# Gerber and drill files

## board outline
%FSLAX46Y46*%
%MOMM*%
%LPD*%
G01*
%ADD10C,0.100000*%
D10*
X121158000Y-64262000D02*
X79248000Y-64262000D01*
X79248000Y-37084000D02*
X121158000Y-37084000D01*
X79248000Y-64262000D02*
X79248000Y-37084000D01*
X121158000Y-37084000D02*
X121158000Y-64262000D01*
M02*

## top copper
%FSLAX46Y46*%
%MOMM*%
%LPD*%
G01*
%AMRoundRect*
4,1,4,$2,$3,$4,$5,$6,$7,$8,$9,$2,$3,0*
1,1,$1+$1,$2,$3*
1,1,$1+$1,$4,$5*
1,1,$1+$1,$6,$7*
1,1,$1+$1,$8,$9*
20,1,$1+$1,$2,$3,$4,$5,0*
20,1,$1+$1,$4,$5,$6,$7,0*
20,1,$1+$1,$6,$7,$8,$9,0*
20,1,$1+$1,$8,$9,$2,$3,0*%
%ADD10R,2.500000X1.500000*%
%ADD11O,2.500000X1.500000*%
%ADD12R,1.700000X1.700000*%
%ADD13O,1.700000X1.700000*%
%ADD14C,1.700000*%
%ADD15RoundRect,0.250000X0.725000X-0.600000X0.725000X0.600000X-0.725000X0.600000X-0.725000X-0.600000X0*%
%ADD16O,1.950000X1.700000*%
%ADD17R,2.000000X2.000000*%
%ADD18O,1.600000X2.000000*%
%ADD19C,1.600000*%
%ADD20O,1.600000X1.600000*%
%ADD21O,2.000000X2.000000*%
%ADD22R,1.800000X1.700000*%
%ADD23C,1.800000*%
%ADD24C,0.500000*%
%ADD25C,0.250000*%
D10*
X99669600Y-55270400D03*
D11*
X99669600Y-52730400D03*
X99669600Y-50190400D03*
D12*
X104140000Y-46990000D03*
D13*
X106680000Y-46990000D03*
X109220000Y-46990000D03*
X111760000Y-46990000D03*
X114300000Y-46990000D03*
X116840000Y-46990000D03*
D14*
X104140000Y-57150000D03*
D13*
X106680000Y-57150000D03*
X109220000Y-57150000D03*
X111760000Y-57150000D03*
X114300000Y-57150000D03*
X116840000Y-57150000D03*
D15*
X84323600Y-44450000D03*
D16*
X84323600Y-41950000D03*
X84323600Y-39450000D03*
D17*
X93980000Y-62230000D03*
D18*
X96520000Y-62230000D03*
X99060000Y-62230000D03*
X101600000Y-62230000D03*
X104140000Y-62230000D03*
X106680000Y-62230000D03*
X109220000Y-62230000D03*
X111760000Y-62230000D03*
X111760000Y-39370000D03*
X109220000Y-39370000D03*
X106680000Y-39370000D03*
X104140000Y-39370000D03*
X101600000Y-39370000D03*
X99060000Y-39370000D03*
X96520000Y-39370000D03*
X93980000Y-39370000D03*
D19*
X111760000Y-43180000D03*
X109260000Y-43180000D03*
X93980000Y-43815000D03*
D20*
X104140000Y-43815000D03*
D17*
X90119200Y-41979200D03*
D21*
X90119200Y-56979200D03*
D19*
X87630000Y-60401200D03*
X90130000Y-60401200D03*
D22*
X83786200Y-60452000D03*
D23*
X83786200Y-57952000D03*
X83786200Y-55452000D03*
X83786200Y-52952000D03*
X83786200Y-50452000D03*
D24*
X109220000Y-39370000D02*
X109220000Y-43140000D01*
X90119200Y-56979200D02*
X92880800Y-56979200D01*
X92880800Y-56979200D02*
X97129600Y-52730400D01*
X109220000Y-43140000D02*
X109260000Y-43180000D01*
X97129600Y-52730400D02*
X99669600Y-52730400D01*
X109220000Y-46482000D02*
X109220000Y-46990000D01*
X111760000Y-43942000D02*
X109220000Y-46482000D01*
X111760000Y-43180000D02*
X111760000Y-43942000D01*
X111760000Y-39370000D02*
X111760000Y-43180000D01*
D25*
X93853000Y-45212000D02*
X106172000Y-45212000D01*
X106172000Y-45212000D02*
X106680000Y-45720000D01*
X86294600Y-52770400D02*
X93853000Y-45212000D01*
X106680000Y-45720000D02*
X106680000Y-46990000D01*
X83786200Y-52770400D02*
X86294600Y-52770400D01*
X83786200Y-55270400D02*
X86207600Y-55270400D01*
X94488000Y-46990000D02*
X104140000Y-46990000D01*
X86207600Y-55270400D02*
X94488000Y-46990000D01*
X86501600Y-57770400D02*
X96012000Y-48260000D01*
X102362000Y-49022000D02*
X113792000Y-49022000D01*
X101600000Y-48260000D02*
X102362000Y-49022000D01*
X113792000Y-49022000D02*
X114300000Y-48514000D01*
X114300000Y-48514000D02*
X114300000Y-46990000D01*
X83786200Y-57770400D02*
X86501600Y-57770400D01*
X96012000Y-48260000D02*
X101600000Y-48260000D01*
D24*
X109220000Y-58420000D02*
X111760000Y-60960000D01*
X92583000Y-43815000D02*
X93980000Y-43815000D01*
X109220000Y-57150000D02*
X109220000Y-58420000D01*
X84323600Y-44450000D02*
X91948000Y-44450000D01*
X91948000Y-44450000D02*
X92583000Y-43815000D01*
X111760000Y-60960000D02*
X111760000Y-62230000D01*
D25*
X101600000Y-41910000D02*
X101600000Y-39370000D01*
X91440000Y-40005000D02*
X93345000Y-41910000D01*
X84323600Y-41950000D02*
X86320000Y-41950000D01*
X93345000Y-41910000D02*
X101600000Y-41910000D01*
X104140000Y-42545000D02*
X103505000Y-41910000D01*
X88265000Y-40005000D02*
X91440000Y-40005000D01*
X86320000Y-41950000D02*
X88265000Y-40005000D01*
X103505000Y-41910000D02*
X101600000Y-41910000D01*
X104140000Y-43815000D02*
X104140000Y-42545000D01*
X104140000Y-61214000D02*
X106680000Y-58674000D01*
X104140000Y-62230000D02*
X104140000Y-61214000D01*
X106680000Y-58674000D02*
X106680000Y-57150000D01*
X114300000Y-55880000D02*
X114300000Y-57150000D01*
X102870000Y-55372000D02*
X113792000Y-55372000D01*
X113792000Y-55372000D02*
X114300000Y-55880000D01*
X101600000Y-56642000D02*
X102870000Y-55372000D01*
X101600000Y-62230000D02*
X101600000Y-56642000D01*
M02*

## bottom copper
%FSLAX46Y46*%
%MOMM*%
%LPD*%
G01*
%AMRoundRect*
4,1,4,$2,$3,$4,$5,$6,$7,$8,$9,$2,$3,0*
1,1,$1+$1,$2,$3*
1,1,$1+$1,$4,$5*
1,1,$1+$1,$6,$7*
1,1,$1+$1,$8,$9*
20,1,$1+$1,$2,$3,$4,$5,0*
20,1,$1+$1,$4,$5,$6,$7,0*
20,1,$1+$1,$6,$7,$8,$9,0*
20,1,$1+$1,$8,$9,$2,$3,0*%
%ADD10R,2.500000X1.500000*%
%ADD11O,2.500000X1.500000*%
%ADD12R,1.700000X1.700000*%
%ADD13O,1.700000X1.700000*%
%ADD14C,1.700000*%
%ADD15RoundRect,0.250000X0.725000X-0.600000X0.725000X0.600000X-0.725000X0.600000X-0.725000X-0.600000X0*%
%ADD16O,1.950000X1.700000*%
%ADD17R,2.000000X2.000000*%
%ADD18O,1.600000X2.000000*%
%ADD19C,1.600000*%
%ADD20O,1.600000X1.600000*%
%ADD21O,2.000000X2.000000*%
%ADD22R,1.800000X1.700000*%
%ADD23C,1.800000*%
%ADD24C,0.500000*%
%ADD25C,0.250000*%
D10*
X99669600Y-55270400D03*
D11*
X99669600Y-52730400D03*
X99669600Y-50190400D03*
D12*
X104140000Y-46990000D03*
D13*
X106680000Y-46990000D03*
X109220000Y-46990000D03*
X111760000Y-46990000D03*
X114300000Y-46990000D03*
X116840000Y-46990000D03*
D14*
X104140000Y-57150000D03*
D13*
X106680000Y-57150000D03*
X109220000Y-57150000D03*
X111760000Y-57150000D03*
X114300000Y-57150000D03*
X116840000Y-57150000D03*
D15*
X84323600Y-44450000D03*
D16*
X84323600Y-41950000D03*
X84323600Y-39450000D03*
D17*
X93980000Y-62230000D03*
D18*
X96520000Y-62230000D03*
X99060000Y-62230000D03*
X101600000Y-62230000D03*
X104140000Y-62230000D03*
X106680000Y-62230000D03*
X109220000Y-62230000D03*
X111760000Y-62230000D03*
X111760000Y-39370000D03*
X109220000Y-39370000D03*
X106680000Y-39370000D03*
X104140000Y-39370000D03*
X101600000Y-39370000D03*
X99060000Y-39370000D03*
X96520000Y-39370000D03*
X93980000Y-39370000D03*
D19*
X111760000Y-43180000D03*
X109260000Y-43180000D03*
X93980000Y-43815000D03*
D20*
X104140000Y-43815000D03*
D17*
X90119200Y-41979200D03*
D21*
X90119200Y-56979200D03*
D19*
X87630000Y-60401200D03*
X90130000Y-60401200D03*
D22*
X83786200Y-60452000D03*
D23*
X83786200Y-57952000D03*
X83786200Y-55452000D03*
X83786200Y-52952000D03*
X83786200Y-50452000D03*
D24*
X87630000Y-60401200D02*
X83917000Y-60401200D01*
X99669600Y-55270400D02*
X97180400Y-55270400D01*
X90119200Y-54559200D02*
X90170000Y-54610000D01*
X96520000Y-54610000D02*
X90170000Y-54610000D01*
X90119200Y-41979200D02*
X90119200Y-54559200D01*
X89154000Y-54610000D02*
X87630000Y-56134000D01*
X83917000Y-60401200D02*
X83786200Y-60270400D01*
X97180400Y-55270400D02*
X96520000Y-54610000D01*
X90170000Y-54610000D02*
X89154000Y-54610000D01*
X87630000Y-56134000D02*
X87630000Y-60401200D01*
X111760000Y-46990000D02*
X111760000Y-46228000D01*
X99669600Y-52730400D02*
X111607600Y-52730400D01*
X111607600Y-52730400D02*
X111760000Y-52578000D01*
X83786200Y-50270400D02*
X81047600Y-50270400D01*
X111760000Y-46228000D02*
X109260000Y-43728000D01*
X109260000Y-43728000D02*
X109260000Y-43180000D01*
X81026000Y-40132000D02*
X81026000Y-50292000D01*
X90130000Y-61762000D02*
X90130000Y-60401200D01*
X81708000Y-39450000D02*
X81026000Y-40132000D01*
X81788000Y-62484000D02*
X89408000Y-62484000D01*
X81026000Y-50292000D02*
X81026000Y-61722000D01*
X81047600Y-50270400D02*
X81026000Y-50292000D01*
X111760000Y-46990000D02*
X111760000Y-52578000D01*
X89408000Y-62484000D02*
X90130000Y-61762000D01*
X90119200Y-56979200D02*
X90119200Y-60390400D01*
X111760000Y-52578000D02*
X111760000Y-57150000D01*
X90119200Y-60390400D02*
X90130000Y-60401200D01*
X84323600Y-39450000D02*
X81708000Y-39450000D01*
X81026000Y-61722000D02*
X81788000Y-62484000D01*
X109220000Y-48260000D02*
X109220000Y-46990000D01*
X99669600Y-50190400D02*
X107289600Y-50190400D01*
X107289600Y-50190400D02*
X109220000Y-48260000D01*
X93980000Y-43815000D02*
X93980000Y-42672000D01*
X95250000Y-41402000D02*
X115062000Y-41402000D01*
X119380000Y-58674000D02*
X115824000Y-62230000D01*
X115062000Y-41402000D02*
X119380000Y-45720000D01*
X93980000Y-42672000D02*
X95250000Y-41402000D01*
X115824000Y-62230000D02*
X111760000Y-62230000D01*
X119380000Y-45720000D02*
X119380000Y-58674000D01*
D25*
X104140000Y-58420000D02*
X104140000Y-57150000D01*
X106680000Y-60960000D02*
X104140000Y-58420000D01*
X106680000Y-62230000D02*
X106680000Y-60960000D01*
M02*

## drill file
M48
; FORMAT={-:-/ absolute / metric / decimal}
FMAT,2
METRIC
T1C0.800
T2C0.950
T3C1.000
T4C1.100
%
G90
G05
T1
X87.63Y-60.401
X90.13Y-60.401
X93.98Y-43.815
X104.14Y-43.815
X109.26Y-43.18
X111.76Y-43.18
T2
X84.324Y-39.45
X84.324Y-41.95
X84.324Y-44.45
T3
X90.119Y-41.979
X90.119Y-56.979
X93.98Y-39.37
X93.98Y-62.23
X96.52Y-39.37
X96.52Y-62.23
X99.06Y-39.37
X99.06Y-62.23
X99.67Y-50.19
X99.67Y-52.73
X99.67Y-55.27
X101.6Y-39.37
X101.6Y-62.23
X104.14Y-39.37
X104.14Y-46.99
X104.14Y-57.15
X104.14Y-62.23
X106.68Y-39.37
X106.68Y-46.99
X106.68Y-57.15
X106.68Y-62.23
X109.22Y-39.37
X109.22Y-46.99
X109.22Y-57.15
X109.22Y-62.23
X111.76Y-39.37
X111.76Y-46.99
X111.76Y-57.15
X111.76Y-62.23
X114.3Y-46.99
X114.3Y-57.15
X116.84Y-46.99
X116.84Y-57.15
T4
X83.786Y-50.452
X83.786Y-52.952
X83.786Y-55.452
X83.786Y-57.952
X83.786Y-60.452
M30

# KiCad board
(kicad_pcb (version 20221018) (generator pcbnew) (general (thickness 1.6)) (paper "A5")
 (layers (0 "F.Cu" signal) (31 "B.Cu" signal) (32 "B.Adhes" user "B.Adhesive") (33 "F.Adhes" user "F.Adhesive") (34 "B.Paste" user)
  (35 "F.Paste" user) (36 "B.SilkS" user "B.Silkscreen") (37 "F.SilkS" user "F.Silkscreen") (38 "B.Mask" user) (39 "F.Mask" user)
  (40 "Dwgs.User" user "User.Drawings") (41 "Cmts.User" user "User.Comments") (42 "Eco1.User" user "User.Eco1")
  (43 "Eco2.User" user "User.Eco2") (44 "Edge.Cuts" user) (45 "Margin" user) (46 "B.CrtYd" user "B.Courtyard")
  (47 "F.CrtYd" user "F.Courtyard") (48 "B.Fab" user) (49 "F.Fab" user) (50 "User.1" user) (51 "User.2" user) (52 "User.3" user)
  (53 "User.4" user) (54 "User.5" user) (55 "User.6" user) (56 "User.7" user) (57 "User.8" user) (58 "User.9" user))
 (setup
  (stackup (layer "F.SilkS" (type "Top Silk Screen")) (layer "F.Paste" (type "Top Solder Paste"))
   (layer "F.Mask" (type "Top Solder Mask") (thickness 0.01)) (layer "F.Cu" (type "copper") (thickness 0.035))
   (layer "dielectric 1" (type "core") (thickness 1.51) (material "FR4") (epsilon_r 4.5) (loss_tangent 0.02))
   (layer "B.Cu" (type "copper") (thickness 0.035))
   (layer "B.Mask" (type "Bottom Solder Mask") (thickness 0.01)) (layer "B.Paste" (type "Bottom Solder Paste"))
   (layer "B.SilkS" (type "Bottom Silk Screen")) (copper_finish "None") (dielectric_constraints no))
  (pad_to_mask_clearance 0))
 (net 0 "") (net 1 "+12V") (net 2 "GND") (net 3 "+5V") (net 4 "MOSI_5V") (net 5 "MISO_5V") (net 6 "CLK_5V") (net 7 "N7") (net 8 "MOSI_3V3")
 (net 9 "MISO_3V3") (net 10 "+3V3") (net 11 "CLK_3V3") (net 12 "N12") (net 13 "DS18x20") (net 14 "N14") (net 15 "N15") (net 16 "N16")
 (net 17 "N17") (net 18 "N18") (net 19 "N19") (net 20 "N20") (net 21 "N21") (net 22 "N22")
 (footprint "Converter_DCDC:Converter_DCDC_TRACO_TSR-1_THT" (layer "F.Cu") (at 99.6696 55.2704 90)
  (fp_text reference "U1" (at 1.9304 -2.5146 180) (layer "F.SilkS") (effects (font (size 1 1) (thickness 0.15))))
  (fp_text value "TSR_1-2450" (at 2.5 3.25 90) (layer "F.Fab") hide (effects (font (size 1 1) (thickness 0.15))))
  (pad "1" thru_hole rect (at 0 0 90) (size 1.5 2.5) (drill 1) (layers "*.Cu" "*.Mask") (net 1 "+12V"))
  (pad "2" thru_hole oval (at 2.54 0 90) (size 1.5 2.5) (drill 1) (layers "*.Cu" "*.Mask") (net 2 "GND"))
  (pad "3" thru_hole oval (at 5.08 0 90) (size 1.5 2.5) (drill 1) (layers "*.Cu" "*.Mask") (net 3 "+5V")))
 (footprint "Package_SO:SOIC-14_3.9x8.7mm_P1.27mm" (layer "F.Cu") (at 110.49 52.07 90)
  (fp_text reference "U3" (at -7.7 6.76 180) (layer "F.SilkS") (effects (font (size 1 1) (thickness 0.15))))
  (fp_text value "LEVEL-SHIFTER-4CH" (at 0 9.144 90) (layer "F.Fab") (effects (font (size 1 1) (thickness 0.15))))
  (pad "1" thru_hole rect (at 5.08 -6.35 90) (size 1.7 1.7) (drill 1) (layers "*.Cu" "*.Mask") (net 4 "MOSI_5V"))
  (pad "2" thru_hole oval (at 5.08 -3.81 90) (size 1.7 1.7) (drill 1) (layers "*.Cu" "*.Mask") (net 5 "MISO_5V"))
  (pad "3" thru_hole oval (at 5.08 -1.27 90) (size 1.7 1.7) (drill 1) (layers "*.Cu" "*.Mask") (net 3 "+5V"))
  (pad "4" thru_hole oval (at 5.08 1.27 90) (size 1.7 1.7) (drill 1) (layers "*.Cu" "*.Mask") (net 2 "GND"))
  (pad "5" thru_hole oval (at 5.08 3.81 90) (size 1.7 1.7) (drill 1) (layers "*.Cu" "*.Mask") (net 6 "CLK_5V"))
  (pad "6" thru_hole oval (at 5.08 6.35 90) (size 1.7 1.7) (drill 1) (layers "*.Cu" "*.Mask") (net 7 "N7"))
  (pad "7" thru_hole circle (at -5.08 -6.35 90) (size 1.7 1.7) (drill 1) (layers "*.Cu" "*.Mask") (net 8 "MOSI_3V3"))
  (pad "8" thru_hole oval (at -5.08 -3.81 90) (size 1.7 1.7) (drill 1) (layers "*.Cu" "*.Mask") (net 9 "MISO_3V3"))
  (pad "9" thru_hole oval (at -5.08 -1.27 90) (size 1.7 1.7) (drill 1) (layers "*.Cu" "*.Mask") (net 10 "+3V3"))
  (pad "10" thru_hole oval (at -5.08 1.27 90) (size 1.7 1.7) (drill 1) (layers "*.Cu" "*.Mask") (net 2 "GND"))
  (pad "11" thru_hole oval (at -5.08 3.81 90) (size 1.7 1.7) (drill 1) (layers "*.Cu" "*.Mask") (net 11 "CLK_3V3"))
  (pad "12" thru_hole oval (at -5.08 6.35 90) (size 1.7 1.7) (drill 1) (layers "*.Cu" "*.Mask") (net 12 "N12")))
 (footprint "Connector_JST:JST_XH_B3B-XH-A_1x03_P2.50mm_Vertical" (layer "F.Cu") (at 84.3236 44.45 90)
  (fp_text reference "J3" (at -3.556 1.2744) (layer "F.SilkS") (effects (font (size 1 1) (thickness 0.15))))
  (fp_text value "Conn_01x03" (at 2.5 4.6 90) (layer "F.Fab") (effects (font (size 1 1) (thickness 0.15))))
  (pad "1" thru_hole roundrect (at 0 0 90) (size 1.7 1.95) (drill 0.95) (layers "*.Cu" "*.Mask") (roundrect_rratio 0.1470588235)
   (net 10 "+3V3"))
  (pad "2" thru_hole oval (at 2.5 0 90) (size 1.7 1.95) (drill 0.95) (layers "*.Cu" "*.Mask") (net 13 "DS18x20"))
  (pad "3" thru_hole oval (at 5 0 90) (size 1.7 1.95) (drill 0.95) (layers "*.Cu" "*.Mask") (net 2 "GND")))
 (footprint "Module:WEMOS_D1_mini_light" (layer "F.Cu") (at 93.98 62.23 90)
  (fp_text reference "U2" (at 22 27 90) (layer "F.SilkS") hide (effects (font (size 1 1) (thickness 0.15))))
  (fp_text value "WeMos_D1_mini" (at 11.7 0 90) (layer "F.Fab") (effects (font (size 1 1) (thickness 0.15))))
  (pad "1" thru_hole rect (at 0 0 90) (size 2 2) (drill 1) (layers "*.Cu" "*.Mask") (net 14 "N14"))
  (pad "2" thru_hole oval (at 0 2.54 90) (size 2 1.6) (drill 1) (layers "*.Cu" "*.Mask") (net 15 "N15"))
  (pad "3" thru_hole oval (at 0 5.08 90) (size 2 1.6) (drill 1) (layers "*.Cu" "*.Mask") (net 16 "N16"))
  (pad "4" thru_hole oval (at 0 7.62 90) (size 2 1.6) (drill 1) (layers "*.Cu" "*.Mask") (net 11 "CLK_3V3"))
  (pad "5" thru_hole oval (at 0 10.16 90) (size 2 1.6) (drill 1) (layers "*.Cu" "*.Mask") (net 9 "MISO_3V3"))
  (pad "6" thru_hole oval (at 0 12.7 90) (size 2 1.6) (drill 1) (layers "*.Cu" "*.Mask") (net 8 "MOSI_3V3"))
  (pad "7" thru_hole oval (at 0 15.24 90) (size 2 1.6) (drill 1) (layers "*.Cu" "*.Mask") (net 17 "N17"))
  (pad "8" thru_hole oval (at 0 17.78 90) (size 2 1.6) (drill 1) (layers "*.Cu" "*.Mask") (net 10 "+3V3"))
  (pad "9" thru_hole oval (at 22.86 17.78 90) (size 2 1.6) (drill 1) (layers "*.Cu" "*.Mask") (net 3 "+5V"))
  (pad "10" thru_hole oval (at 22.86 15.24 90) (size 2 1.6) (drill 1) (layers "*.Cu" "*.Mask") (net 2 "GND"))
  (pad "11" thru_hole oval (at 22.86 12.7 90) (size 2 1.6) (drill 1) (layers "*.Cu" "*.Mask") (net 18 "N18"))
  (pad "12" thru_hole oval (at 22.86 10.16 90) (size 2 1.6) (drill 1) (layers "*.Cu" "*.Mask") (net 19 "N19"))
  (pad "13" thru_hole oval (at 22.86 7.62 90) (size 2 1.6) (drill 1) (layers "*.Cu" "*.Mask") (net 13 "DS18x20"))
  (pad "14" thru_hole oval (at 22.86 5.08 90) (size 2 1.6) (drill 1) (layers "*.Cu" "*.Mask") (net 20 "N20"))
  (pad "15" thru_hole oval (at 22.86 2.54 90) (size 2 1.6) (drill 1) (layers "*.Cu" "*.Mask") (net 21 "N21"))
  (pad "16" thru_hole oval (at 22.86 0 90) (size 2 1.6) (drill 1) (layers "*.Cu" "*.Mask") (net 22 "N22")))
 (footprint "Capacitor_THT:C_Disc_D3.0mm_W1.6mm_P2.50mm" (layer "F.Cu") (at 111.76 43.18 180)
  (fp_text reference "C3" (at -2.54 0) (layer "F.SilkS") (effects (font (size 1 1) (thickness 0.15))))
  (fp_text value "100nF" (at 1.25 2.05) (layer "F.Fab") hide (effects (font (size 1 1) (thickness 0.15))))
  (pad "1" thru_hole circle (at 0 0 180) (size 1.6 1.6) (drill 0.8) (layers "*.Cu" "*.Mask") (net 3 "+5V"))
  (pad "2" thru_hole circle (at 2.5 0 180) (size 1.6 1.6) (drill 0.8) (layers "*.Cu" "*.Mask") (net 2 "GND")))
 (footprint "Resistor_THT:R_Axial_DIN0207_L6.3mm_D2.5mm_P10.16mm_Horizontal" (layer "F.Cu") (at 93.98 43.815)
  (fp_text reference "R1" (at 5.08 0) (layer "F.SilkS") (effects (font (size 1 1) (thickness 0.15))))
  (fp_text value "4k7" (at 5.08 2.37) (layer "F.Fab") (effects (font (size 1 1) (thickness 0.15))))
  (pad "1" thru_hole circle (at 0 0) (size 1.6 1.6) (drill 0.8) (layers "*.Cu" "*.Mask") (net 10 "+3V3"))
  (pad "2" thru_hole oval (at 10.16 0) (size 1.6 1.6) (drill 0.8) (layers "*.Cu" "*.Mask") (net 13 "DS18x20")))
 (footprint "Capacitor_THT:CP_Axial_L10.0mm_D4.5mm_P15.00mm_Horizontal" (layer "F.Cu") (at 90.1192 41.9792 -90)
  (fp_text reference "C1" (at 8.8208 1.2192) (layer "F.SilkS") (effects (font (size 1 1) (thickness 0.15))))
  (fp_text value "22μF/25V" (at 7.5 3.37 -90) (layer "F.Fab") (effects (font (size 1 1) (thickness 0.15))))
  (pad "1" thru_hole rect (at 0 0 270) (size 2 2) (drill 1) (layers "*.Cu" "*.Mask") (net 1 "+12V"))
  (pad "2" thru_hole oval (at 15 0 270) (size 2 2) (drill 1) (layers "*.Cu" "*.Mask") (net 2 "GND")))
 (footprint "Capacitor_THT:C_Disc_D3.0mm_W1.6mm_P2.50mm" (layer "F.Cu") (at 87.63 60.4012)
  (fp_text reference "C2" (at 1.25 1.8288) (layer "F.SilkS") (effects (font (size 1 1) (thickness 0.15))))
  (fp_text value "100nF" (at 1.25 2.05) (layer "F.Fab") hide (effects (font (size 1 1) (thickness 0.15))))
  (pad "1" thru_hole circle (at 0 0) (size 1.6 1.6) (drill 0.8) (layers "*.Cu" "*.Mask") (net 1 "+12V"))
  (pad "2" thru_hole circle (at 2.5 0) (size 1.6 1.6) (drill 0.8) (layers "*.Cu" "*.Mask") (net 2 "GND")))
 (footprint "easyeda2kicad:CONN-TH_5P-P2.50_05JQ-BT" (layer "B.Cu") (at 83.7862 55.452 -90)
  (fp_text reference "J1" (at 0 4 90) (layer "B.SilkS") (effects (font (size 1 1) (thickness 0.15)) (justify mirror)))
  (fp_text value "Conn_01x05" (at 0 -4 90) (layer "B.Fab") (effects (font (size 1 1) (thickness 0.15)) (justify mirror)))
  (pad "1" thru_hole rect (at 5 0 90) (size 1.7 1.8) (drill 1.100023) (layers "*.Cu" "*.Paste" "*.Mask") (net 2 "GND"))
  (pad "2" thru_hole circle (at 2.5 0 90) (size 1.8 1.8) (drill 1.100023) (layers "*.Cu" "*.Paste" "*.Mask") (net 5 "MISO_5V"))
  (pad "3" thru_hole circle (at 0 0 90) (size 1.8 1.8) (drill 1.100023) (layers "*.Cu" "*.Paste" "*.Mask") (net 4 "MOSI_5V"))
  (pad "4" thru_hole circle (at -2.5 0 90) (size 1.8 1.8) (drill 1.100023) (layers "*.Cu" "*.Paste" "*.Mask") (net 6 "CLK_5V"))
  (pad "5" thru_hole circle (at -5 0 90) (size 1.8 1.8) (drill 1.100023) (layers "*.Cu" "*.Paste" "*.Mask") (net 1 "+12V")))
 (gr_line (start 121.158 64.262) (end 79.248 64.262) (stroke (width 0.1) (type solid)) (layer "Edge.Cuts"))
 (gr_line (start 79.248 37.084) (end 121.158 37.084) (stroke (width 0.1) (type solid)) (layer "Edge.Cuts"))
 (gr_line (start 79.248 64.262) (end 79.248 37.084) (stroke (width 0.1) (type solid)) (layer "Edge.Cuts"))
 (gr_line (start 121.158 37.084) (end 121.158 64.262) (stroke (width 0.1) (type solid)) (layer "Edge.Cuts"))
 (segment (start 87.63 60.4012) (end 83.917 60.4012) (width 0.5) (layer "B.Cu") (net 1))
 (segment (start 99.6696 55.2704) (end 97.1804 55.2704) (width 0.5) (layer "B.Cu") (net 1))
 (segment (start 90.1192 54.5592) (end 90.17 54.61) (width 0.5) (layer "B.Cu") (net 1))
 (segment (start 96.52 54.61) (end 90.17 54.61) (width 0.5) (layer "B.Cu") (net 1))
 (segment (start 90.1192 41.9792) (end 90.1192 54.5592) (width 0.5) (layer "B.Cu") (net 1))
 (segment (start 89.154 54.61) (end 87.63 56.134) (width 0.5) (layer "B.Cu") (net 1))
 (segment (start 83.917 60.4012) (end 83.7862 60.2704) (width 0.5) (layer "B.Cu") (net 1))
 (segment (start 97.1804 55.2704) (end 96.52 54.61) (width 0.5) (layer "B.Cu") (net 1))
 (segment (start 90.17 54.61) (end 89.154 54.61) (width 0.5) (layer "B.Cu") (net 1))
 (segment (start 87.63 56.134) (end 87.63 60.4012) (width 0.5) (layer "B.Cu") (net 1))
 (segment (start 109.22 39.37) (end 109.22 43.14) (width 0.5) (layer "F.Cu") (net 2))
 (segment (start 90.1192 56.9792) (end 92.8808 56.9792) (width 0.5) (layer "F.Cu") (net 2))
 (segment (start 92.8808 56.9792) (end 97.1296 52.7304) (width 0.5) (layer "F.Cu") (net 2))
 (segment (start 109.22 43.14) (end 109.26 43.18) (width 0.5) (layer "F.Cu") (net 2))
 (segment (start 97.1296 52.7304) (end 99.6696 52.7304) (width 0.5) (layer "F.Cu") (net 2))
 (segment (start 111.76 46.99) (end 111.76 46.228) (width 0.5) (layer "B.Cu") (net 2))
 (segment (start 99.6696 52.7304) (end 111.6076 52.7304) (width 0.5) (layer "B.Cu") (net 2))
 (segment (start 111.6076 52.7304) (end 111.76 52.578) (width 0.5) (layer "B.Cu") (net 2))
 (segment (start 83.7862 50.2704) (end 81.0476 50.2704) (width 0.5) (layer "B.Cu") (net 2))
 (segment (start 111.76 46.228) (end 109.26 43.728) (width 0.5) (layer "B.Cu") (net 2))
 (segment (start 109.26 43.728) (end 109.26 43.18) (width 0.5) (layer "B.Cu") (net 2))
 (segment (start 81.026 40.132) (end 81.026 50.292) (width 0.5) (layer "B.Cu") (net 2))
 (segment (start 90.13 61.762) (end 90.13 60.4012) (width 0.5) (layer "B.Cu") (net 2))
 (segment (start 81.708 39.45) (end 81.026 40.132) (width 0.5) (layer "B.Cu") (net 2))
 (segment (start 81.788 62.484) (end 89.408 62.484) (width 0.5) (layer "B.Cu") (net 2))
 (segment (start 81.026 50.292) (end 81.026 61.722) (width 0.5) (layer "B.Cu") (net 2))
 (segment (start 81.0476 50.2704) (end 81.026 50.292) (width 0.5) (layer "B.Cu") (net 2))
 (segment (start 111.76 46.99) (end 111.76 52.578) (width 0.5) (layer "B.Cu") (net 2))
 (segment (start 89.408 62.484) (end 90.13 61.762) (width 0.5) (layer "B.Cu") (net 2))
 (segment (start 90.1192 56.9792) (end 90.1192 60.3904) (width 0.5) (layer "B.Cu") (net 2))
 (segment (start 111.76 52.578) (end 111.76 57.15) (width 0.5) (layer "B.Cu") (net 2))
 (segment (start 90.1192 60.3904) (end 90.13 60.4012) (width 0.5) (layer "B.Cu") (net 2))
 (segment (start 84.3236 39.45) (end 81.708 39.45) (width 0.5) (layer "B.Cu") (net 2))
 (segment (start 81.026 61.722) (end 81.788 62.484) (width 0.5) (layer "B.Cu") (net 2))
 (segment (start 109.22 46.482) (end 109.22 46.99) (width 0.5) (layer "F.Cu") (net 3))
 (segment (start 111.76 43.942) (end 109.22 46.482) (width 0.5) (layer "F.Cu") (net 3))
 (segment (start 111.76 43.18) (end 111.76 43.942) (width 0.5) (layer "F.Cu") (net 3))
 (segment (start 111.76 39.37) (end 111.76 43.18) (width 0.5) (layer "F.Cu") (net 3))
 (segment (start 109.22 48.26) (end 109.22 46.99) (width 0.5) (layer "B.Cu") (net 3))
 (segment (start 99.6696 50.1904) (end 107.2896 50.1904) (width 0.5) (layer "B.Cu") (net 3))
 (segment (start 107.2896 50.1904) (end 109.22 48.26) (width 0.5) (layer "B.Cu") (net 3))
 (segment (start 93.853 45.212) (end 106.172 45.212) (width 0.25) (layer "F.Cu") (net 5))
 (segment (start 106.172 45.212) (end 106.68 45.72) (width 0.25) (layer "F.Cu") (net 5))
 (segment (start 86.2946 52.7704) (end 93.853 45.212) (width 0.25) (layer "F.Cu") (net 5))
 (segment (start 106.68 45.72) (end 106.68 46.99) (width 0.25) (layer "F.Cu") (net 5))
 (segment (start 83.7862 52.7704) (end 86.2946 52.7704) (width 0.25) (layer "F.Cu") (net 5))
 (segment (start 83.7862 55.2704) (end 86.2076 55.2704) (width 0.25) (layer "F.Cu") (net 4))
 (segment (start 94.488 46.99) (end 104.14 46.99) (width 0.25) (layer "F.Cu") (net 4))
 (segment (start 86.2076 55.2704) (end 94.488 46.99) (width 0.25) (layer "F.Cu") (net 4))
 (segment (start 86.5016 57.7704) (end 96.012 48.26) (width 0.25) (layer "F.Cu") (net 6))
 (segment (start 102.362 49.022) (end 113.792 49.022) (width 0.25) (layer "F.Cu") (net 6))
 (segment (start 101.6 48.26) (end 102.362 49.022) (width 0.25) (layer "F.Cu") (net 6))
 (segment (start 113.792 49.022) (end 114.3 48.514) (width 0.25) (layer "F.Cu") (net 6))
 (segment (start 114.3 48.514) (end 114.3 46.99) (width 0.25) (layer "F.Cu") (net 6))
 (segment (start 83.7862 57.7704) (end 86.5016 57.7704) (width 0.25) (layer "F.Cu") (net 6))
 (segment (start 96.012 48.26) (end 101.6 48.26) (width 0.25) (layer "F.Cu") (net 6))
 (segment (start 109.22 58.42) (end 111.76 60.96) (width 0.5) (layer "F.Cu") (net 10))
 (segment (start 92.583 43.815) (end 93.98 43.815) (width 0.5) (layer "F.Cu") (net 10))
 (segment (start 109.22 57.15) (end 109.22 58.42) (width 0.5) (layer "F.Cu") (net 10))
 (segment (start 84.3236 44.45) (end 91.948 44.45) (width 0.5) (layer "F.Cu") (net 10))
 (segment (start 91.948 44.45) (end 92.583 43.815) (width 0.5) (layer "F.Cu") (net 10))
 (segment (start 111.76 60.96) (end 111.76 62.23) (width 0.5) (layer "F.Cu") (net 10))
 (segment (start 93.98 43.815) (end 93.98 42.672) (width 0.5) (layer "B.Cu") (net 10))
 (segment (start 95.25 41.402) (end 115.062 41.402) (width 0.5) (layer "B.Cu") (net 10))
 (segment (start 119.38 58.674) (end 115.824 62.23) (width 0.5) (layer "B.Cu") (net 10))
 (segment (start 115.062 41.402) (end 119.38 45.72) (width 0.5) (layer "B.Cu") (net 10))
 (segment (start 93.98 42.672) (end 95.25 41.402) (width 0.5) (layer "B.Cu") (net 10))
 (segment (start 115.824 62.23) (end 111.76 62.23) (width 0.5) (layer "B.Cu") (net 10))
 (segment (start 119.38 45.72) (end 119.38 58.674) (width 0.5) (layer "B.Cu") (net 10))
 (segment (start 101.6 41.91) (end 101.6 39.37) (width 0.25) (layer "F.Cu") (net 13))
 (segment (start 91.44 40.005) (end 93.345 41.91) (width 0.25) (layer "F.Cu") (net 13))
 (segment (start 84.3236 41.95) (end 86.32 41.95) (width 0.25) (layer "F.Cu") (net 13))
 (segment (start 93.345 41.91) (end 101.6 41.91) (width 0.25) (layer "F.Cu") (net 13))
 (segment (start 104.14 42.545) (end 103.505 41.91) (width 0.25) (layer "F.Cu") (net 13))
 (segment (start 88.265 40.005) (end 91.44 40.005) (width 0.25) (layer "F.Cu") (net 13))
 (segment (start 86.32 41.95) (end 88.265 40.005) (width 0.25) (layer "F.Cu") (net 13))
 (segment (start 103.505 41.91) (end 101.6 41.91) (width 0.25) (layer "F.Cu") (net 13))
 (segment (start 104.14 43.815) (end 104.14 42.545) (width 0.25) (layer "F.Cu") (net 13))
 (segment (start 104.14 58.42) (end 104.14 57.15) (width 0.25) (layer "B.Cu") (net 8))
 (segment (start 106.68 60.96) (end 104.14 58.42) (width 0.25) (layer "B.Cu") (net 8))
 (segment (start 106.68 62.23) (end 106.68 60.96) (width 0.25) (layer "B.Cu") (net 8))
 (segment (start 104.14 61.214) (end 106.68 58.674) (width 0.25) (layer "F.Cu") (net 9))
 (segment (start 104.14 62.23) (end 104.14 61.214) (width 0.25) (layer "F.Cu") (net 9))
 (segment (start 106.68 58.674) (end 106.68 57.15) (width 0.25) (layer "F.Cu") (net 9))
 (segment (start 114.3 55.88) (end 114.3 57.15) (width 0.25) (layer "F.Cu") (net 11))
 (segment (start 102.87 55.372) (end 113.792 55.372) (width 0.25) (layer "F.Cu") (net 11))
 (segment (start 113.792 55.372) (end 114.3 55.88) (width 0.25) (layer "F.Cu") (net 11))
 (segment (start 101.6 56.642) (end 102.87 55.372) (width 0.25) (layer "F.Cu") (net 11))
 (segment (start 101.6 62.23) (end 101.6 56.642) (width 0.25) (layer "F.Cu") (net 11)))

